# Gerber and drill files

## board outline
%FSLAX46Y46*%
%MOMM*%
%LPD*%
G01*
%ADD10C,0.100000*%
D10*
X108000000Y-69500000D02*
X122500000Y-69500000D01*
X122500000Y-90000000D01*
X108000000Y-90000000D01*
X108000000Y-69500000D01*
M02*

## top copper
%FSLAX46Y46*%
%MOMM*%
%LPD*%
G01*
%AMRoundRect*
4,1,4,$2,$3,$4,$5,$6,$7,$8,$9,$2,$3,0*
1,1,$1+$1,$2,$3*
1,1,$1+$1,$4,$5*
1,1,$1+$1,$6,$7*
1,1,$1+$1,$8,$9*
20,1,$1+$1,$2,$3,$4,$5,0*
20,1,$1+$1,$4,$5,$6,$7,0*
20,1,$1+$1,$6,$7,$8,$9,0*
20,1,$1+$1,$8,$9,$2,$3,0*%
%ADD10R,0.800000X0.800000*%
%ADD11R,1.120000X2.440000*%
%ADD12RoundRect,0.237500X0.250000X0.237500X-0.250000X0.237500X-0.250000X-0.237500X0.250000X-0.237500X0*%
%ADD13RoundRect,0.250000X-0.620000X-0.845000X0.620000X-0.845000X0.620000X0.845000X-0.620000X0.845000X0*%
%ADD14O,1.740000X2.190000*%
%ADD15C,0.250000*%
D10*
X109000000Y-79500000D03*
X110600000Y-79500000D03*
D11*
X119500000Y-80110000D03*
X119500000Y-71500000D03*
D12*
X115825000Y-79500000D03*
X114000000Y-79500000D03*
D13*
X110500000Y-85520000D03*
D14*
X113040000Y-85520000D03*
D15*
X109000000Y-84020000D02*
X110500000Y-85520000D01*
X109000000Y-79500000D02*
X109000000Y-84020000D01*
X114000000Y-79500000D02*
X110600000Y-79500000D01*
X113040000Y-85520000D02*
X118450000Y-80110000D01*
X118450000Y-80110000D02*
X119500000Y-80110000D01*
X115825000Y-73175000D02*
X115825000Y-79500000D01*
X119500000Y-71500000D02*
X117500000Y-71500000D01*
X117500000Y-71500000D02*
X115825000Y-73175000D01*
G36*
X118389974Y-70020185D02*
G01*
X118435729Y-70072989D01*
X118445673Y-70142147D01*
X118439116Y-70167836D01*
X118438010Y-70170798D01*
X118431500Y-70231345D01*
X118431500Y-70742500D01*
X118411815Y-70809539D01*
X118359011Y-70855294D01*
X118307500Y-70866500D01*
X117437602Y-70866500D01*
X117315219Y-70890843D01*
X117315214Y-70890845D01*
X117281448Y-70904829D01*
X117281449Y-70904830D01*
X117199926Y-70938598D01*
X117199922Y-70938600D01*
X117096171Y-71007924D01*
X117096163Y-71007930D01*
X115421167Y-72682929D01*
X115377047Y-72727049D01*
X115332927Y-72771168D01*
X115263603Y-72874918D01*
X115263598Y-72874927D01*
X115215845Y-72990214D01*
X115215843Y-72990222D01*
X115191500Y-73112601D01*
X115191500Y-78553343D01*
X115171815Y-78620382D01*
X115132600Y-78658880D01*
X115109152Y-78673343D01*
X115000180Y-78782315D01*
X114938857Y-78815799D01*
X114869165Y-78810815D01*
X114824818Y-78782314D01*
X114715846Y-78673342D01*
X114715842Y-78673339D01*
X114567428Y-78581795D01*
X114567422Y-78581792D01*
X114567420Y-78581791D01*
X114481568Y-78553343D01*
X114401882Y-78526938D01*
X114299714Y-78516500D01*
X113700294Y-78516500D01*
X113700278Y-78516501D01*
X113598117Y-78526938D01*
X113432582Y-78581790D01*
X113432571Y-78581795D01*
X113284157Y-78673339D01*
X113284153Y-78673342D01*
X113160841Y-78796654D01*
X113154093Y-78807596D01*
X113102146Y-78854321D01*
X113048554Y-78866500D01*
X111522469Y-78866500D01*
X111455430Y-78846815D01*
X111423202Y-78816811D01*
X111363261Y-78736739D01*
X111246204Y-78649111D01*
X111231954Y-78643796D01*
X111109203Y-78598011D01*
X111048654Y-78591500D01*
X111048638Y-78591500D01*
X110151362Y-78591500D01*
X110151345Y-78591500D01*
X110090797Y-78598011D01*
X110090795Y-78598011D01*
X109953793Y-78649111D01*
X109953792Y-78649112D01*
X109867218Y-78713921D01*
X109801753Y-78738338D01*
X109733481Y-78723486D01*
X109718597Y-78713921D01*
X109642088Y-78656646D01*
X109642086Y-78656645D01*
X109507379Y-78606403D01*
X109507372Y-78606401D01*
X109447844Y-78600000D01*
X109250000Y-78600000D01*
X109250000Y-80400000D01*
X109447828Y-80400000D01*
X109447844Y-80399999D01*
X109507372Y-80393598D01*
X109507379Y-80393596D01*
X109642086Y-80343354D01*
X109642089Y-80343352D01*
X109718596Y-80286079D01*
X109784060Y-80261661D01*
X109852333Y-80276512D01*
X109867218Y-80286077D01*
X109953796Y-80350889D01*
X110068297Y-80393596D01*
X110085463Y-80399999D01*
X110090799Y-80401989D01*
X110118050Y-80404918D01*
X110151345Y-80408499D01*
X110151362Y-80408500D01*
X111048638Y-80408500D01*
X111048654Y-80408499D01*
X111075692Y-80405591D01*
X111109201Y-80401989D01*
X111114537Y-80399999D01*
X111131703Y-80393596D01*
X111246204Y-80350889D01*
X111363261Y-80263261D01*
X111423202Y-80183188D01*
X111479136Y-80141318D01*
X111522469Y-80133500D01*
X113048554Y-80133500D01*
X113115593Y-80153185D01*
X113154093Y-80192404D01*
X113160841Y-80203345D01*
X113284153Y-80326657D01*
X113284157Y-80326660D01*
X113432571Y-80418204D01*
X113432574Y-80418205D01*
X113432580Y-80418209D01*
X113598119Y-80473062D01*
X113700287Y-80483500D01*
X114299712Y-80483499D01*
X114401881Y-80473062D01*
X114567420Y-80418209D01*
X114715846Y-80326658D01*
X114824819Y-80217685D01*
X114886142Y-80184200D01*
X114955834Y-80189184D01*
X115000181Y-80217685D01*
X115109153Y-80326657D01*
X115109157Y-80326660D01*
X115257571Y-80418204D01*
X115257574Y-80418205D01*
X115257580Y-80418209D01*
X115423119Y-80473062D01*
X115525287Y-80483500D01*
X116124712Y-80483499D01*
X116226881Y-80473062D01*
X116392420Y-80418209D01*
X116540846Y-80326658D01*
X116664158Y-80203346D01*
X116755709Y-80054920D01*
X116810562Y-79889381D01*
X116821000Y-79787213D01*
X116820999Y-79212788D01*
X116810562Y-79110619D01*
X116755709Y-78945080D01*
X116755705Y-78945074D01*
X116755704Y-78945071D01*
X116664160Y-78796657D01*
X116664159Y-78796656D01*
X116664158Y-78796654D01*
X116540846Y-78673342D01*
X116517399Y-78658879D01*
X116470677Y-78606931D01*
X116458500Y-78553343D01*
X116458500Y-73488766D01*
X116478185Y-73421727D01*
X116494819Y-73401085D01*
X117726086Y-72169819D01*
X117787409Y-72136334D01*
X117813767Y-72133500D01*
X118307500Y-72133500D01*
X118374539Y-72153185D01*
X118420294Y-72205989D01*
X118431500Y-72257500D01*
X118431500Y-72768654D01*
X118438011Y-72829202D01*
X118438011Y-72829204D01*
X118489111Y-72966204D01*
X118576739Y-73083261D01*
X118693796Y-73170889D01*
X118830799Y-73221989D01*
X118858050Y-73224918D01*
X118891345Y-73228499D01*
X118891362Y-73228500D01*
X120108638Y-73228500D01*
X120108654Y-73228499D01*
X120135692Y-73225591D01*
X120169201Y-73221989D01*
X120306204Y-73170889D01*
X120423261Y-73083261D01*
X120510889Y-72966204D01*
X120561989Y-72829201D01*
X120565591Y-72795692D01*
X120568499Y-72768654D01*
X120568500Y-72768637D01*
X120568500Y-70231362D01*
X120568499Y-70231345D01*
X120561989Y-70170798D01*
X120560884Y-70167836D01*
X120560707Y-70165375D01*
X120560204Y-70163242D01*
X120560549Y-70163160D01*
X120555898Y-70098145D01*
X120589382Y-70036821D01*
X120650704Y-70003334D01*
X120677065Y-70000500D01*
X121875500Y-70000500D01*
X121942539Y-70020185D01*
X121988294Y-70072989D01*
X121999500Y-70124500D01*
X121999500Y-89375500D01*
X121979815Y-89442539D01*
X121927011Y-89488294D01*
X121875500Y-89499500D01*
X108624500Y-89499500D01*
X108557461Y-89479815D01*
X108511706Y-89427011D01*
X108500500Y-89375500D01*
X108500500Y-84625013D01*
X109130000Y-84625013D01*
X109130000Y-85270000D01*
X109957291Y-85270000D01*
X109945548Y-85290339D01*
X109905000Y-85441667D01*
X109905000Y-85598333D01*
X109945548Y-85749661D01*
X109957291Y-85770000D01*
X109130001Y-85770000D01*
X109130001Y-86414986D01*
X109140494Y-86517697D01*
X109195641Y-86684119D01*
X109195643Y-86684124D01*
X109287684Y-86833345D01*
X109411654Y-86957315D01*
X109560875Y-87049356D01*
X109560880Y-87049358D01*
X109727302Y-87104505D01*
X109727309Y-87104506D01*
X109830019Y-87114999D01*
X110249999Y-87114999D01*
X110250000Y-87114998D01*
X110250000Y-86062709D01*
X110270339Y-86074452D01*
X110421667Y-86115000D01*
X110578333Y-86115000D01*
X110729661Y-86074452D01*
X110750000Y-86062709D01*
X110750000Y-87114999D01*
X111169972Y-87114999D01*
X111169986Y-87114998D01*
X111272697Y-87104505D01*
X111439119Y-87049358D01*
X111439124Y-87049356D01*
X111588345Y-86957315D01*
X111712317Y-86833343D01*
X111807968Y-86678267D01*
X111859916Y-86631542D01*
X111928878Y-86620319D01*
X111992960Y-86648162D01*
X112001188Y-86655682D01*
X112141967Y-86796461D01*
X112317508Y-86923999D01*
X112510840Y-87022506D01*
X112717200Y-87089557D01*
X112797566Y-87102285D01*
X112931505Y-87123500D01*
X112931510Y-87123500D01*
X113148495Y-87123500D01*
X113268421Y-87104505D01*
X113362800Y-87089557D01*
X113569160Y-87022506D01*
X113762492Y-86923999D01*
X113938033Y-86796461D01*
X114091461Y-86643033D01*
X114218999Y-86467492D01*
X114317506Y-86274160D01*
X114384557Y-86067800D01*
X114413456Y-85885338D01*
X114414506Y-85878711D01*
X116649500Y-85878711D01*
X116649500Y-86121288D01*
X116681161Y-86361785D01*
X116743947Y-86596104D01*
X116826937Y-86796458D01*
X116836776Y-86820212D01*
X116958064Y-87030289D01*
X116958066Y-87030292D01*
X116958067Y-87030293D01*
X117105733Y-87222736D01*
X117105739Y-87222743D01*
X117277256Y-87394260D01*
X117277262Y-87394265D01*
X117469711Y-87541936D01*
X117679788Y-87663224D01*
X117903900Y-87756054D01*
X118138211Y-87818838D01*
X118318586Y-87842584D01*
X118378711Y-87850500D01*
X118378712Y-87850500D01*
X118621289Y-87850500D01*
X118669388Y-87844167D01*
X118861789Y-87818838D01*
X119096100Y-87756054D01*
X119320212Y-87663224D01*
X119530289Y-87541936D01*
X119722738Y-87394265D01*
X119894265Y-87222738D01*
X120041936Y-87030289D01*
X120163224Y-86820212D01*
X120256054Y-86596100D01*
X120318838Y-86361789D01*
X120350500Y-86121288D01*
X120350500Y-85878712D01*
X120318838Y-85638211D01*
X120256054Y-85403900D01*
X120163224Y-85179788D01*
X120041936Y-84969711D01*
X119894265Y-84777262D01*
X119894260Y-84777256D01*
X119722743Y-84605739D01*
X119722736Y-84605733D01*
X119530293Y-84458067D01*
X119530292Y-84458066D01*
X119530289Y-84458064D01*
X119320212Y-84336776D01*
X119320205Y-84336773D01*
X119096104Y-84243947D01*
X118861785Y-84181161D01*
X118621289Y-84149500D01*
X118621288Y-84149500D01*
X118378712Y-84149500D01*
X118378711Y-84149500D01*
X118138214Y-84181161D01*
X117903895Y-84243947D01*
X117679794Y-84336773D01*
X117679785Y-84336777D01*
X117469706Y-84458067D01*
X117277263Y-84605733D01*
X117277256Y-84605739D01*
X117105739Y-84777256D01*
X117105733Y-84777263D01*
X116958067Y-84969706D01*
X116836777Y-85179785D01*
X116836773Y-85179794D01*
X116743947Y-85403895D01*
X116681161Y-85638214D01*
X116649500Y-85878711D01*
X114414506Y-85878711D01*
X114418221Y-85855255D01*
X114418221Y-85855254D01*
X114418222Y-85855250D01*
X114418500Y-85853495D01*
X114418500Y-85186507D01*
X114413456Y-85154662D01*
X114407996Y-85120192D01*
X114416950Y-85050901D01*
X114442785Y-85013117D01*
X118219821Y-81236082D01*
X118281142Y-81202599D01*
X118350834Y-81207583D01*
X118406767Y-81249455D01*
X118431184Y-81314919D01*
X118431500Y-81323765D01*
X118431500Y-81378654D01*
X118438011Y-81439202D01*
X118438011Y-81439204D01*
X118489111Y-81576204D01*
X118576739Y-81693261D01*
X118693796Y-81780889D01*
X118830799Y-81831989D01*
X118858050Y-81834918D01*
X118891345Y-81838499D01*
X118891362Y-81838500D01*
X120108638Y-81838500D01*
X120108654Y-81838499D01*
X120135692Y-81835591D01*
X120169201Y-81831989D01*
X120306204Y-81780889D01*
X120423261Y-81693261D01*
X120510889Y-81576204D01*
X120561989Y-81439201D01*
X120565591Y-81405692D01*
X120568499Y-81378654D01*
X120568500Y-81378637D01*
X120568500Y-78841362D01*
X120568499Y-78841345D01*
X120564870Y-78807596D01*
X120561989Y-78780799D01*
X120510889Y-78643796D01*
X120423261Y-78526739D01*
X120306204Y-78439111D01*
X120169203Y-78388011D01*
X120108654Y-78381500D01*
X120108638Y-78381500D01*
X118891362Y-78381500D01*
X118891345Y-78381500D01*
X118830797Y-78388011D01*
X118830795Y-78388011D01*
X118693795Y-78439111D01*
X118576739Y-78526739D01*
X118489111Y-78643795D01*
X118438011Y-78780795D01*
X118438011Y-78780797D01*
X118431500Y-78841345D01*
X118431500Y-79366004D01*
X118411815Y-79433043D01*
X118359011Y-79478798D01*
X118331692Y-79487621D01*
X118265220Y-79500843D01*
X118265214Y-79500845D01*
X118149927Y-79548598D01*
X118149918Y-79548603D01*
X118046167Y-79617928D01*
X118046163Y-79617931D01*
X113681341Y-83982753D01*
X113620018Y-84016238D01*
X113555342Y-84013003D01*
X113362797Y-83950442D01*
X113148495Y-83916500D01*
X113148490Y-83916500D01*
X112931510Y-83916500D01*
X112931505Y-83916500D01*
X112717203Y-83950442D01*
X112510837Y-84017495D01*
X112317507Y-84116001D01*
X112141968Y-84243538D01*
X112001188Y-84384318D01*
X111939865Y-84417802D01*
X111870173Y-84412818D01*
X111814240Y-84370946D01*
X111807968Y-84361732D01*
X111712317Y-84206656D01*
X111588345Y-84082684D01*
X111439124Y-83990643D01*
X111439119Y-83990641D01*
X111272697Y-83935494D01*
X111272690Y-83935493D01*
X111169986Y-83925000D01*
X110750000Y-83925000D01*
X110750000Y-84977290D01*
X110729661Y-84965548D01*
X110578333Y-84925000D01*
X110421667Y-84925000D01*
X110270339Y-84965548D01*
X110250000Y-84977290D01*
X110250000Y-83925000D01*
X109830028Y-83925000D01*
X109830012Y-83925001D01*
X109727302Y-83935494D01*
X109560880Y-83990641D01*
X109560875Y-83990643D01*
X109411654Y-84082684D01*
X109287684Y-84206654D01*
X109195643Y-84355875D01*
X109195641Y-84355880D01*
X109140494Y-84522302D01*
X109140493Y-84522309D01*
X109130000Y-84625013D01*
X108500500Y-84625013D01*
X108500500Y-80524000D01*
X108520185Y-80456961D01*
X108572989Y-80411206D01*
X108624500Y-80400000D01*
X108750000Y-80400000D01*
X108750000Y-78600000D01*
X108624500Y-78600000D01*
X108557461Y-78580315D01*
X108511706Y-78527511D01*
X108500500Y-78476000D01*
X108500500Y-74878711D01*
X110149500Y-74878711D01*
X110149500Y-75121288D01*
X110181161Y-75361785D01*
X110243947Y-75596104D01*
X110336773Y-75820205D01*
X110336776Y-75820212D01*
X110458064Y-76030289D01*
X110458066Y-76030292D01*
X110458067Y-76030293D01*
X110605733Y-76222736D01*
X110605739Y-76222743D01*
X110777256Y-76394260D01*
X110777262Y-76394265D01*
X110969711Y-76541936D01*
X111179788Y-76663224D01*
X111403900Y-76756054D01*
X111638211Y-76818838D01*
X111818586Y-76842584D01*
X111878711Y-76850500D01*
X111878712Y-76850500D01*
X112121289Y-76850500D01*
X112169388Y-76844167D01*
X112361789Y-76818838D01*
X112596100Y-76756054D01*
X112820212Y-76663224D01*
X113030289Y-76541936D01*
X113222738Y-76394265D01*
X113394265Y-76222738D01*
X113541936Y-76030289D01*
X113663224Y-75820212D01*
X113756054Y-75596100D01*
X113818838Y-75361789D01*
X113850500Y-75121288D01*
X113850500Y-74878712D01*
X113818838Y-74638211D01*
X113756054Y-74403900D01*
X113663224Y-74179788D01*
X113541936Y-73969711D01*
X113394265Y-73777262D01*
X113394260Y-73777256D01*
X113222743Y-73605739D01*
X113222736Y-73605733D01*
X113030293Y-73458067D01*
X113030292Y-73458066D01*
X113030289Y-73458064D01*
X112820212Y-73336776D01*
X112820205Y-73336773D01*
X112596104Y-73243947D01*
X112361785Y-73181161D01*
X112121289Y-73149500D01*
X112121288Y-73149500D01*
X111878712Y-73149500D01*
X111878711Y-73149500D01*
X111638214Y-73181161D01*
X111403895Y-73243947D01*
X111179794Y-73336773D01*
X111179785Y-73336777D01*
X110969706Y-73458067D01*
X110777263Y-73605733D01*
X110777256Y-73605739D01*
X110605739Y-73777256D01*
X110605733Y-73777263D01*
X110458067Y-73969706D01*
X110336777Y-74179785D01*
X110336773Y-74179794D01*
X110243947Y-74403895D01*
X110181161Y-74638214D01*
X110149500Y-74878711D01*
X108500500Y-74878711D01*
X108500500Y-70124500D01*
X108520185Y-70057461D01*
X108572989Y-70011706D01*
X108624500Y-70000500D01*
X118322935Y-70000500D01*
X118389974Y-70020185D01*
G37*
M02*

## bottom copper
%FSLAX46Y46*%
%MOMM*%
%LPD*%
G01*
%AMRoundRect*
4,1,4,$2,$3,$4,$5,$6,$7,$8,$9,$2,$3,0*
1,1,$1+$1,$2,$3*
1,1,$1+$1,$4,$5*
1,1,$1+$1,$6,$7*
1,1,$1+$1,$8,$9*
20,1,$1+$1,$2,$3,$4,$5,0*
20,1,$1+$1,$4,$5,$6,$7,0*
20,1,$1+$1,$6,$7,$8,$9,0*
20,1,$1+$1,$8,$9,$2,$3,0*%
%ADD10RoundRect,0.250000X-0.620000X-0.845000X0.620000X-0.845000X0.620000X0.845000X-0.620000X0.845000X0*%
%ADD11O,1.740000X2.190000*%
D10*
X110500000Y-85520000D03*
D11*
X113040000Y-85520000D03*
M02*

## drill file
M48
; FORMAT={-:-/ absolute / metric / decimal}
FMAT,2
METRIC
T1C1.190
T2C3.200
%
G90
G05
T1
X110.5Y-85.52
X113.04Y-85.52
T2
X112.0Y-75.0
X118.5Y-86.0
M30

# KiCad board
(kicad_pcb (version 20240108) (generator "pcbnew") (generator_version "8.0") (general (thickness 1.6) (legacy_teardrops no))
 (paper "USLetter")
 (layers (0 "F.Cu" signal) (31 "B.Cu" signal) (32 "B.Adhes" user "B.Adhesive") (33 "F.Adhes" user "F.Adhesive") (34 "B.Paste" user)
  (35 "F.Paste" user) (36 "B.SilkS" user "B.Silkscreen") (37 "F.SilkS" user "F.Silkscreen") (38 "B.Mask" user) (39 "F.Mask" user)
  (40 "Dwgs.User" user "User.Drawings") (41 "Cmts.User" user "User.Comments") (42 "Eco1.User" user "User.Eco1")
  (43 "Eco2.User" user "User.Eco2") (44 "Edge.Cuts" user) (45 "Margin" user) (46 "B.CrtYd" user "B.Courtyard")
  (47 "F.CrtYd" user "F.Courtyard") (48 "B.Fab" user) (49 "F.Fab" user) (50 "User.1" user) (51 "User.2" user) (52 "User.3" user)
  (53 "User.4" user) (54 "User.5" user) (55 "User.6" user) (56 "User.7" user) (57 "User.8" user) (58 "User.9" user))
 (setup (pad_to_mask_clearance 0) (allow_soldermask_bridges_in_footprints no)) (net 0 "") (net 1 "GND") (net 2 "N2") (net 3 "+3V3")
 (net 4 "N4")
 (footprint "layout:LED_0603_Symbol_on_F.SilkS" (layer "F.Cu") (at 109.8 79.5)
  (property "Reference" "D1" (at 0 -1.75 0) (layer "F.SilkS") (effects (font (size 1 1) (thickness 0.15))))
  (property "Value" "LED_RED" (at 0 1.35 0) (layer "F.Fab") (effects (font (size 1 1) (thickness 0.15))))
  (pad "1" smd rect (at -0.8 0 180) (size 0.8 0.8) (layers "F.Cu" "F.Paste" "F.Mask") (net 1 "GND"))
  (pad "2" smd rect (at 0.8 0 180) (size 0.8 0.8) (layers "F.Cu" "F.Paste" "F.Mask") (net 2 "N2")))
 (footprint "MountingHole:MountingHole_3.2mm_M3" (layer "F.Cu") (at 112 75)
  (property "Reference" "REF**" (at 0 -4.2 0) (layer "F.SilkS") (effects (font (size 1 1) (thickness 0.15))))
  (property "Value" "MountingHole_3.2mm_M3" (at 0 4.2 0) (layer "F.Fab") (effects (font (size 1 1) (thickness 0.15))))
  (pad "" np_thru_hole circle (at 0 0) (size 3.2 3.2) (drill 3.2) (layers "*.Cu" "*.Mask")))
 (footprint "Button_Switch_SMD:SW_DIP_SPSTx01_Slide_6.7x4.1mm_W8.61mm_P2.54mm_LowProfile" (layer "F.Cu") (at 119.5 75.805 90)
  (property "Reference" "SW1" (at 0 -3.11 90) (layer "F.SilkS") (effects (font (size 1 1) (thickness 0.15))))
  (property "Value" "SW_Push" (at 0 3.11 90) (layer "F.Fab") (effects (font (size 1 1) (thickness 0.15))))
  (pad "1" smd rect (at -4.305 0 90) (size 2.44 1.12) (layers "F.Cu" "F.Paste" "F.Mask") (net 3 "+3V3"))
  (pad "2" smd rect (at 4.305 0 90) (size 2.44 1.12) (layers "F.Cu" "F.Paste" "F.Mask") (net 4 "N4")))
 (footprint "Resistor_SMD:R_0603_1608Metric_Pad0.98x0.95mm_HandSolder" (layer "F.Cu") (at 114.9125 79.5 180)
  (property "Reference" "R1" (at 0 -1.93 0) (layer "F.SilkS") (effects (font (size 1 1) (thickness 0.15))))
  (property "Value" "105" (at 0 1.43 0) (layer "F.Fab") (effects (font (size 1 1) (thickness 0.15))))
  (pad "1" smd roundrect (at -0.9125 0 180) (size 0.975 0.95) (layers "F.Cu" "F.Paste" "F.Mask") (roundrect_rratio 0.25) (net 4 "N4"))
  (pad "2" smd roundrect (at 0.9125 0 180) (size 0.975 0.95) (layers "F.Cu" "F.Paste" "F.Mask") (roundrect_rratio 0.25) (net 2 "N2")))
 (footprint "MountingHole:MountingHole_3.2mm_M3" (layer "F.Cu") (at 118.5 86)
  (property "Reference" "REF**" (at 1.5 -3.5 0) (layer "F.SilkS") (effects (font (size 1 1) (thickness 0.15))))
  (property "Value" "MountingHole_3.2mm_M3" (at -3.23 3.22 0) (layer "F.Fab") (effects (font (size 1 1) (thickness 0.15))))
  (pad "" np_thru_hole circle (at 0 0) (size 3.2 3.2) (drill 3.2) (layers "*.Cu" "*.Mask")))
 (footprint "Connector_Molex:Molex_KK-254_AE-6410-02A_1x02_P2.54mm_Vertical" (layer "F.Cu") (at 110.5 85.52)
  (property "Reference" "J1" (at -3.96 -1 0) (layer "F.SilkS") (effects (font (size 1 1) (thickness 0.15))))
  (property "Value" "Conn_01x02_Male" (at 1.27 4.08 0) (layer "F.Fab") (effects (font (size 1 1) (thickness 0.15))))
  (pad "1" thru_hole roundrect (at 0 0) (size 1.74 2.19) (drill 1.19) (layers "*.Cu" "*.Mask") (remove_unused_layers no)
   (roundrect_rratio 0.143678) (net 1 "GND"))
  (pad "2" thru_hole oval (at 2.54 0) (size 1.74 2.19) (drill 1.19) (layers "*.Cu" "*.Mask") (remove_unused_layers no) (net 3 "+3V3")))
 (gr_rect (start 108 69.5) (end 122.5 90) (stroke (width 0.1) (type default)) (fill none) (layer "Edge.Cuts"))
 (segment (start 109 84.02) (end 110.5 85.52) (width 0.25) (layer "F.Cu") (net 1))
 (segment (start 109 79.5) (end 109 84.02) (width 0.25) (layer "F.Cu") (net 1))
 (segment (start 114 79.5) (end 110.6 79.5) (width 0.25) (layer "F.Cu") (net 2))
 (segment (start 113.04 85.52) (end 118.45 80.11) (width 0.25) (layer "F.Cu") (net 3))
 (segment (start 118.45 80.11) (end 119.5 80.11) (width 0.25) (layer "F.Cu") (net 3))
 (segment (start 115.825 73.175) (end 115.825 79.5) (width 0.25) (layer "F.Cu") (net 4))
 (segment (start 119.5 71.5) (end 117.5 71.5) (width 0.25) (layer "F.Cu") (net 4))
 (segment (start 117.5 71.5) (end 115.825 73.175) (width 0.25) (layer "F.Cu") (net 4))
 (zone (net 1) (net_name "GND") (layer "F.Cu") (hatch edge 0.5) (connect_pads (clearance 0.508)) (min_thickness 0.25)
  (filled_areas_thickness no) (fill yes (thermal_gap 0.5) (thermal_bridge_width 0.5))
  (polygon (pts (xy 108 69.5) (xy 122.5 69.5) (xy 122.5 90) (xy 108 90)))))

